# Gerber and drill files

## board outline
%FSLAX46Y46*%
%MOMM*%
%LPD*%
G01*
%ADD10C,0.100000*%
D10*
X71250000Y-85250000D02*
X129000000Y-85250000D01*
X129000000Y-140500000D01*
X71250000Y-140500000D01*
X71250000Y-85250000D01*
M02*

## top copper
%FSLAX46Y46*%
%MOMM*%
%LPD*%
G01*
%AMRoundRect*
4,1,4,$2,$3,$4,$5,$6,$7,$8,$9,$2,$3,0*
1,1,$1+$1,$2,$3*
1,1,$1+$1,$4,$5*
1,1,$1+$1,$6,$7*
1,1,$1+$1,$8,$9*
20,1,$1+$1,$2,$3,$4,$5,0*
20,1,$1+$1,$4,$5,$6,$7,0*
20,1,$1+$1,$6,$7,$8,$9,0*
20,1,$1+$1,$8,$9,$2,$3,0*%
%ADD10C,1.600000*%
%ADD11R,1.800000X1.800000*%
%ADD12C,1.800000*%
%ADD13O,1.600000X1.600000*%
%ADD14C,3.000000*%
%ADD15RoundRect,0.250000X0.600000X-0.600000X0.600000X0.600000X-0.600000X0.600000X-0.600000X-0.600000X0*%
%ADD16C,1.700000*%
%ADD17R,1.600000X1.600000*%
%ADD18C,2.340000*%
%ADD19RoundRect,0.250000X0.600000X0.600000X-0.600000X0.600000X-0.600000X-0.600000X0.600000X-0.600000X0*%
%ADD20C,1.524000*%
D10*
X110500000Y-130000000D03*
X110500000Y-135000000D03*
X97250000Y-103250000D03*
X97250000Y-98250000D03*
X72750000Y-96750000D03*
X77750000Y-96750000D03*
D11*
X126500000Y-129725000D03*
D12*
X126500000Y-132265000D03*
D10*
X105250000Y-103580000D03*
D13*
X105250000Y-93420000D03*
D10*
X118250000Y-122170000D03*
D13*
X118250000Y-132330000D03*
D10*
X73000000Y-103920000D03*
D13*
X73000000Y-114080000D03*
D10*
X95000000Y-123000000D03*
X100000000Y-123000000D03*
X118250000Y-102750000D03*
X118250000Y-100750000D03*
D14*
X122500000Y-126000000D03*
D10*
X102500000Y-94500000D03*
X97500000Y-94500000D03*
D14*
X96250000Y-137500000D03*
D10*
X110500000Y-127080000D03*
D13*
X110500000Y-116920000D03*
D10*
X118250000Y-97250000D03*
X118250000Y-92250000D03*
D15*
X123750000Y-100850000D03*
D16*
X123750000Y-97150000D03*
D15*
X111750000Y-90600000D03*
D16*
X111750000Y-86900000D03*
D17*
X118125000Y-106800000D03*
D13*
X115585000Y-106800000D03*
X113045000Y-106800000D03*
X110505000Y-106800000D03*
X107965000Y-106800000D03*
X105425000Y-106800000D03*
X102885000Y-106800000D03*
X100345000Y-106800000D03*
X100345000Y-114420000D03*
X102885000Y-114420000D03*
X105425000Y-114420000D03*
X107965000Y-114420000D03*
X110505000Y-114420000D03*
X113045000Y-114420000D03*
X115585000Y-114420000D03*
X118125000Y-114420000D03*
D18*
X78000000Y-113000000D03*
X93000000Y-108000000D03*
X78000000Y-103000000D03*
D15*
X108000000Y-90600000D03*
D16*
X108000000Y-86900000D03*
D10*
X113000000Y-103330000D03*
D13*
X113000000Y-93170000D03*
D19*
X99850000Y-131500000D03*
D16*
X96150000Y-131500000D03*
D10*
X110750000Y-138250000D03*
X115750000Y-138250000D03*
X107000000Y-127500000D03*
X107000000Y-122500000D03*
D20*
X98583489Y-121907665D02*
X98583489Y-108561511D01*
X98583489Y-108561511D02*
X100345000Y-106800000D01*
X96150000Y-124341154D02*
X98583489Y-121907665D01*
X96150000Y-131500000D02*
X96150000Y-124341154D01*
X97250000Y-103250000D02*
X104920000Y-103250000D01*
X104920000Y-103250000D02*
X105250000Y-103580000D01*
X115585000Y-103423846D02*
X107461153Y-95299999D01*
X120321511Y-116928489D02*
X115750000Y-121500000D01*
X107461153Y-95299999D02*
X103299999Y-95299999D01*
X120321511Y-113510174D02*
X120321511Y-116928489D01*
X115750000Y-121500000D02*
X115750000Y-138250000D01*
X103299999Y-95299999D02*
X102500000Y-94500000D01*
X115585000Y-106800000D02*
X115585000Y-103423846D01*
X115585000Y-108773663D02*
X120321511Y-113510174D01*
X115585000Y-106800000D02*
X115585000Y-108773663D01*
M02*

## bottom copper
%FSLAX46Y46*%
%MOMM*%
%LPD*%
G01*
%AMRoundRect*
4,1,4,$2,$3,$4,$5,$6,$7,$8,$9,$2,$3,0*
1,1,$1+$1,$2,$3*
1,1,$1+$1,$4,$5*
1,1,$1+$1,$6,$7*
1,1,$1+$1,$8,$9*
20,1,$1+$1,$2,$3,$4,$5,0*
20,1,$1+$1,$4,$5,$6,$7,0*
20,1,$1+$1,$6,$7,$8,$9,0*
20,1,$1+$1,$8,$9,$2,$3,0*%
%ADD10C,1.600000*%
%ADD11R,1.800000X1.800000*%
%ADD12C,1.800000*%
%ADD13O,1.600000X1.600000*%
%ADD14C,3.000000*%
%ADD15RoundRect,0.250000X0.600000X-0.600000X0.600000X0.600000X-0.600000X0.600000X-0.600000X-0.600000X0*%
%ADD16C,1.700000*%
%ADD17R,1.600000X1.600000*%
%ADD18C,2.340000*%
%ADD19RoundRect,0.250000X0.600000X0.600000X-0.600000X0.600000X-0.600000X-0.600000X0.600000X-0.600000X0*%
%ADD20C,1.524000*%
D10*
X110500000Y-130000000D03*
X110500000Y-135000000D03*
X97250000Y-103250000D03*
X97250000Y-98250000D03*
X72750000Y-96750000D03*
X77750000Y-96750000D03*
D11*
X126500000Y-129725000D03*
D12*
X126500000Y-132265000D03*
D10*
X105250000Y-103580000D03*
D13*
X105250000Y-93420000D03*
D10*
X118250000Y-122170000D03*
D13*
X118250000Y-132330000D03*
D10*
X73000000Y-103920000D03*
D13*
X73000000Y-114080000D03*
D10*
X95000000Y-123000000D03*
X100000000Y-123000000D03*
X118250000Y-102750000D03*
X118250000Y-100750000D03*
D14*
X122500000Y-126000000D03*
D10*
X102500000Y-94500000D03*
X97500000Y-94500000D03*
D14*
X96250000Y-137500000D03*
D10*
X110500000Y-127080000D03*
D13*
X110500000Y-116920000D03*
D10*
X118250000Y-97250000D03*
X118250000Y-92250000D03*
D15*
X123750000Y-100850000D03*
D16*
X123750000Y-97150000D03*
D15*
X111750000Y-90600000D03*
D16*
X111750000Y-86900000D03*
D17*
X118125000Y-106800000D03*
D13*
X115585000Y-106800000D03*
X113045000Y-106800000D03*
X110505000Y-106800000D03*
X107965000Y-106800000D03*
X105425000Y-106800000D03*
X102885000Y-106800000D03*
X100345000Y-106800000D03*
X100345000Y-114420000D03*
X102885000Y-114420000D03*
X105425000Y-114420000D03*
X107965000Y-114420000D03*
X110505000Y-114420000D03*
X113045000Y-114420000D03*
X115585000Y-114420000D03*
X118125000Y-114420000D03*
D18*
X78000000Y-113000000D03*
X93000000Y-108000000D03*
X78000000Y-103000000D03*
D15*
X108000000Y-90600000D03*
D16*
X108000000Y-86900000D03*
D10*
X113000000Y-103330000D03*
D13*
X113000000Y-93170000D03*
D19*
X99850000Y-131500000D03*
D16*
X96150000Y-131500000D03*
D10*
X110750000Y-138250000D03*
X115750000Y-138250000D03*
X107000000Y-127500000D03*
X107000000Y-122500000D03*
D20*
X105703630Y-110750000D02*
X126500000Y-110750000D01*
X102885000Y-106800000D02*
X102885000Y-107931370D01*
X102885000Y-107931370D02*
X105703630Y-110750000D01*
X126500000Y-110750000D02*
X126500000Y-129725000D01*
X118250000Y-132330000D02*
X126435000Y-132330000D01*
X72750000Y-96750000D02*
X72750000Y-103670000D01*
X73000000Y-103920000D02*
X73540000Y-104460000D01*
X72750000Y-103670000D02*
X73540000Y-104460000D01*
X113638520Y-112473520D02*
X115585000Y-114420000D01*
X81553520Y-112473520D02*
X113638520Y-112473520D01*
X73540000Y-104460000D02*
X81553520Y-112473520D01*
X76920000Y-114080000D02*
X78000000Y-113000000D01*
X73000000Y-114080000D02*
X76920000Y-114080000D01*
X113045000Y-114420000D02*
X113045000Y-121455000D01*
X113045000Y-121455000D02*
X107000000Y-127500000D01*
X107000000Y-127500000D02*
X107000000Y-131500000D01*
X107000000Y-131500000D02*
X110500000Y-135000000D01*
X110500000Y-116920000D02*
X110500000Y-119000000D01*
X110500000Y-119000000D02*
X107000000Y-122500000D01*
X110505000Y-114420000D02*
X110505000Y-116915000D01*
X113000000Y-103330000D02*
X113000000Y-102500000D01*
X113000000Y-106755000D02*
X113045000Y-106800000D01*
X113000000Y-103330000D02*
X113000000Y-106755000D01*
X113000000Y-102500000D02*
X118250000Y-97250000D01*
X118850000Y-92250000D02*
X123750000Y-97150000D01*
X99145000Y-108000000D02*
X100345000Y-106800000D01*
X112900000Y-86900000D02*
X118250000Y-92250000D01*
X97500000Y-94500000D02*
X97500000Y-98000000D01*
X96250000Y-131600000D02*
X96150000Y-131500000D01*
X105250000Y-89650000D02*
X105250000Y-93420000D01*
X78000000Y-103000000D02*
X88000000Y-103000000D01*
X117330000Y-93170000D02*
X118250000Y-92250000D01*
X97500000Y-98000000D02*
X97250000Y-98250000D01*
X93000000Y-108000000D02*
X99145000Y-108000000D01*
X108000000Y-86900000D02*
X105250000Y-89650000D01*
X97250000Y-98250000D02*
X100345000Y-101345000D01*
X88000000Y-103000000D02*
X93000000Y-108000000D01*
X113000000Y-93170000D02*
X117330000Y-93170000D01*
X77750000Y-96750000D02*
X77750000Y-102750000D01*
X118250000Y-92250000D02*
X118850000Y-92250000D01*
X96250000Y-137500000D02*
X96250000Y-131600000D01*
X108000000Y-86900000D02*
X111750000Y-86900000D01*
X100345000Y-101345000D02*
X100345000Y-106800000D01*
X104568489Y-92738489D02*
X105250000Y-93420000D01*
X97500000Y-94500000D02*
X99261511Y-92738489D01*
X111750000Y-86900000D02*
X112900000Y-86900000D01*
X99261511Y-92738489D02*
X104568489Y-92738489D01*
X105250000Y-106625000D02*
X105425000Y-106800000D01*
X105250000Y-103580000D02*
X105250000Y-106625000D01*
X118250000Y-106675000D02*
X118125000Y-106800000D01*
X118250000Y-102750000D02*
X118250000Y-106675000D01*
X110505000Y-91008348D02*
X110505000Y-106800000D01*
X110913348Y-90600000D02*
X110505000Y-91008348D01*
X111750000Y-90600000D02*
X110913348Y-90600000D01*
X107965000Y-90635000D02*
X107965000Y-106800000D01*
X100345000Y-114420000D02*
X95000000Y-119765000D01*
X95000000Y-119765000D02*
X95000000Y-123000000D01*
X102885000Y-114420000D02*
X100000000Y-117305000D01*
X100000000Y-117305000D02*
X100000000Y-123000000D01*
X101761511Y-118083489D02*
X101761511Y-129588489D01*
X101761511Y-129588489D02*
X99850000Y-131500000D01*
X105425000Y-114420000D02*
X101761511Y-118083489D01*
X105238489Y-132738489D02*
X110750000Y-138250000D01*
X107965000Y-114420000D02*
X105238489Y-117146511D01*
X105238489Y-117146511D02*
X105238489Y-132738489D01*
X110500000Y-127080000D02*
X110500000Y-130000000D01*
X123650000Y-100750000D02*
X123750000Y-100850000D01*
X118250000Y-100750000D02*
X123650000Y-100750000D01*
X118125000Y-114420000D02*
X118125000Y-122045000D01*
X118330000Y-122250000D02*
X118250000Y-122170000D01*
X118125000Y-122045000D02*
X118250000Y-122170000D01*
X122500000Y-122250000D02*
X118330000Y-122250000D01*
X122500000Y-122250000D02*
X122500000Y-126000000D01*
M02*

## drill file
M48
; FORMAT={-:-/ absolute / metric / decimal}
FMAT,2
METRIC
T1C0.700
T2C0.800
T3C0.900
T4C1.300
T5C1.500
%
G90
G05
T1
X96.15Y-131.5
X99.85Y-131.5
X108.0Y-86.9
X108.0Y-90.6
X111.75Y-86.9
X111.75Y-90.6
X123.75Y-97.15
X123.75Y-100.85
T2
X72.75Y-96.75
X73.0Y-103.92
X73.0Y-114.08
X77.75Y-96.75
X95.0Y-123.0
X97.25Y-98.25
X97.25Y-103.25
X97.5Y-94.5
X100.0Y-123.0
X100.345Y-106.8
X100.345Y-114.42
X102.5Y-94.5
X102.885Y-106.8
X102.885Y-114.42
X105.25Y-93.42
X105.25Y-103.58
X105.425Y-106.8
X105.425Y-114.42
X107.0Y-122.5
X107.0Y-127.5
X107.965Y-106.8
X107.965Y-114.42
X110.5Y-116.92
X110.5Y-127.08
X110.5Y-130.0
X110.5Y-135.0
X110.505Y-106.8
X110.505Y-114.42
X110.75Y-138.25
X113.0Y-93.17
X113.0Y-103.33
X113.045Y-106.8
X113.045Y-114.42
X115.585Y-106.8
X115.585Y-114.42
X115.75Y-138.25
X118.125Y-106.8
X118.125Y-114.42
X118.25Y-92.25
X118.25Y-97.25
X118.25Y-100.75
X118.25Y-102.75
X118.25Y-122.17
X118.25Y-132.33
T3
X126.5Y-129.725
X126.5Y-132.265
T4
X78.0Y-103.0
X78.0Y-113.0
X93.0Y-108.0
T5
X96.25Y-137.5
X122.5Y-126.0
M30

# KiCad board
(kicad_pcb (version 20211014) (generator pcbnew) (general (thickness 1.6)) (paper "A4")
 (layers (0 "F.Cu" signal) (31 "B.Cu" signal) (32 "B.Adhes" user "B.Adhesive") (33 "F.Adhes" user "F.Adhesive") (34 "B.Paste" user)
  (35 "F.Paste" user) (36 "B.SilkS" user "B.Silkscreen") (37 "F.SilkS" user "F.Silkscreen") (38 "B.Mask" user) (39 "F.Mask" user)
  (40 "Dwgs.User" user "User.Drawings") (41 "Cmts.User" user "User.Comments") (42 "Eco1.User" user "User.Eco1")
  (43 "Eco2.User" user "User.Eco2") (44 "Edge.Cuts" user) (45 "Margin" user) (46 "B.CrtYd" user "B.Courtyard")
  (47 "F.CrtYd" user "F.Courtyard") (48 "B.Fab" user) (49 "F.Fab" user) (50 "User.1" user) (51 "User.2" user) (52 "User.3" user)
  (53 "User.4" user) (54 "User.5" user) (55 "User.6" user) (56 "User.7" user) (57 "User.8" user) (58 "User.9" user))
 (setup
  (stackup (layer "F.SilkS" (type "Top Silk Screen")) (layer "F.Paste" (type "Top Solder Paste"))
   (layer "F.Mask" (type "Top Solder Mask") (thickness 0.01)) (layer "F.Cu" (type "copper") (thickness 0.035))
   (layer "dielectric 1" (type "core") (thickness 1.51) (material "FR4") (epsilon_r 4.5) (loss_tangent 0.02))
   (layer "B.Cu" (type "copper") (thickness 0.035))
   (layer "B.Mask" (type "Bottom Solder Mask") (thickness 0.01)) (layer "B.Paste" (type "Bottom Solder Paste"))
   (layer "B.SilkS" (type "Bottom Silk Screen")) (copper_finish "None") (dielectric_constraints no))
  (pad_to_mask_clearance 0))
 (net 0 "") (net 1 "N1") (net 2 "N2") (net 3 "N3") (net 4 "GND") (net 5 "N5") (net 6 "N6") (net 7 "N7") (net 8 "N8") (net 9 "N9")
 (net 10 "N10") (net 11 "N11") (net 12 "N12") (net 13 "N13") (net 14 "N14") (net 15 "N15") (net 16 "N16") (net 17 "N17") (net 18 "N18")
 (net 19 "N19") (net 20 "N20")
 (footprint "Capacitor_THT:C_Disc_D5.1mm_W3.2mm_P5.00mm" (layer "F.Cu") (at 110.5 130 -90)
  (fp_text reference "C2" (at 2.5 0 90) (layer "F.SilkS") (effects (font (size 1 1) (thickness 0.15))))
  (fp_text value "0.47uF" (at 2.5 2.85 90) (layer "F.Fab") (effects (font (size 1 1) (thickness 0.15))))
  (pad "1" thru_hole circle (at 0 0 270) (size 1.6 1.6) (drill 0.8) (layers *.Cu *.Mask) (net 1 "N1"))
  (pad "2" thru_hole circle (at 5 0 270) (size 1.6 1.6) (drill 0.8) (layers *.Cu *.Mask) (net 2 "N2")))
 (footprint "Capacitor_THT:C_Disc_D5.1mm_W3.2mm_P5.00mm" (layer "F.Cu") (at 97.25 103.25 90)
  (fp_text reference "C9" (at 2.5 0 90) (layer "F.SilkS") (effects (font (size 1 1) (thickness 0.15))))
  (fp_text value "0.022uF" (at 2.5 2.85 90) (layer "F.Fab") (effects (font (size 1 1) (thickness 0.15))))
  (pad "1" thru_hole circle (at 0 0 90) (size 1.6 1.6) (drill 0.8) (layers *.Cu *.Mask) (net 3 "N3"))
  (pad "2" thru_hole circle (at 5 0 90) (size 1.6 1.6) (drill 0.8) (layers *.Cu *.Mask) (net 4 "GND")))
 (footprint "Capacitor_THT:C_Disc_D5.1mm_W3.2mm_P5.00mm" (layer "F.Cu") (at 72.75 96.75)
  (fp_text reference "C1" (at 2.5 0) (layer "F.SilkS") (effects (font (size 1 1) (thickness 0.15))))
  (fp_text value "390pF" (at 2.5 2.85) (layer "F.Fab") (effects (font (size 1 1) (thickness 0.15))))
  (pad "1" thru_hole circle (at 0 0) (size 1.6 1.6) (drill 0.8) (layers *.Cu *.Mask) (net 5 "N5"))
  (pad "2" thru_hole circle (at 5 0) (size 1.6 1.6) (drill 0.8) (layers *.Cu *.Mask) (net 4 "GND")))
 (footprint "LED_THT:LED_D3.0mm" (layer "F.Cu") (at 126.5 129.725 -90)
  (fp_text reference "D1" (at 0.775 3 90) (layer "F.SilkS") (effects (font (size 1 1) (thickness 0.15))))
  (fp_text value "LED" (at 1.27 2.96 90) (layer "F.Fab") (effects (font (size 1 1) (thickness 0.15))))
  (pad "1" thru_hole rect (at 0 0 270) (size 1.8 1.8) (drill 0.9) (layers *.Cu *.Mask) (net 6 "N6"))
  (pad "2" thru_hole circle (at 2.54 0 270) (size 1.8 1.8) (drill 0.9) (layers *.Cu *.Mask) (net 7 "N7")))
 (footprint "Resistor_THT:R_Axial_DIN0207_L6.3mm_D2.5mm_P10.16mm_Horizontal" (layer "F.Cu") (at 105.25 103.58 90)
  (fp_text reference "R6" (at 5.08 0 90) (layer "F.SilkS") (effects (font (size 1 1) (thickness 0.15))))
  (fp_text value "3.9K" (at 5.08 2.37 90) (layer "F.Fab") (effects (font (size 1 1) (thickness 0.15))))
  (pad "1" thru_hole circle (at 0 0 90) (size 1.6 1.6) (drill 0.8) (layers *.Cu *.Mask) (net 3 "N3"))
  (pad "2" thru_hole oval (at 10.16 0 90) (size 1.6 1.6) (drill 0.8) (layers *.Cu *.Mask) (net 4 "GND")))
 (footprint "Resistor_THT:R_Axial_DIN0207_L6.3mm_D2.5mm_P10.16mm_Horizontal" (layer "F.Cu") (at 118.25 122.17 -90)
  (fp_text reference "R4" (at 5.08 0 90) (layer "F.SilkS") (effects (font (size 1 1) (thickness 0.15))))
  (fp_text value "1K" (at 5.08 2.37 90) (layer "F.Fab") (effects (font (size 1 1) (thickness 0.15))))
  (pad "1" thru_hole circle (at 0 0 270) (size 1.6 1.6) (drill 0.8) (layers *.Cu *.Mask) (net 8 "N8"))
  (pad "2" thru_hole oval (at 10.16 0 270) (size 1.6 1.6) (drill 0.8) (layers *.Cu *.Mask) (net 7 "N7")))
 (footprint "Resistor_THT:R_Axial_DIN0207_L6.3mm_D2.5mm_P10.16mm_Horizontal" (layer "F.Cu") (at 73 103.92 -90)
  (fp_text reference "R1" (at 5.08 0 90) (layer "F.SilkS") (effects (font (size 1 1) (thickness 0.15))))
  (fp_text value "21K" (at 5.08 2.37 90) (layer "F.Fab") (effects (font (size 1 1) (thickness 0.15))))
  (pad "1" thru_hole circle (at 0 0 270) (size 1.6 1.6) (drill 0.8) (layers *.Cu *.Mask) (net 5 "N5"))
  (pad "2" thru_hole oval (at 10.16 0 270) (size 1.6 1.6) (drill 0.8) (layers *.Cu *.Mask) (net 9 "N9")))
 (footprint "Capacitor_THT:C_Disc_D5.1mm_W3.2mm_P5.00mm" (layer "F.Cu") (at 95 123)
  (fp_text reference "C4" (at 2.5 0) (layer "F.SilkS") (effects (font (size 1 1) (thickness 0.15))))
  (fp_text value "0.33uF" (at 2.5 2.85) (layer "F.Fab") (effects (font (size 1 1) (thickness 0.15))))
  (pad "1" thru_hole circle (at 0 0) (size 1.6 1.6) (drill 0.8) (layers *.Cu *.Mask) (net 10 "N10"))
  (pad "2" thru_hole circle (at 5 0) (size 1.6 1.6) (drill 0.8) (layers *.Cu *.Mask) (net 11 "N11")))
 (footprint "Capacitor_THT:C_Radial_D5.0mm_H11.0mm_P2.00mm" (layer "F.Cu") (at 118.25 102.75 90)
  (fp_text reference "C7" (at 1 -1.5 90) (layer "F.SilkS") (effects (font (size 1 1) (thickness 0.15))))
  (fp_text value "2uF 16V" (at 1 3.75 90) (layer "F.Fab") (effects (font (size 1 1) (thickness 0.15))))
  (pad "1" thru_hole circle (at 0 0 90) (size 1.6 1.6) (drill 0.8) (layers *.Cu *.Mask) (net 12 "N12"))
  (pad "2" thru_hole circle (at 2 0 90) (size 1.6 1.6) (drill 0.8) (layers *.Cu *.Mask) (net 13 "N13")))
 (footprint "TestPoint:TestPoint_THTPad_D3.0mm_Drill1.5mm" (layer "F.Cu") (at 122.5 126)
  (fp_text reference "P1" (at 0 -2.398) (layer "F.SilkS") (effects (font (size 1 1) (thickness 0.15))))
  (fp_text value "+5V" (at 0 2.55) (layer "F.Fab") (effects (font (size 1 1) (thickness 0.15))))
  (pad "1" thru_hole circle (at 0 0) (size 3 3) (drill 1.5) (layers *.Cu *.Mask) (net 8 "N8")))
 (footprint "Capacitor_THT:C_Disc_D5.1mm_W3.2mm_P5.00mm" (layer "F.Cu") (at 102.5 94.5 180)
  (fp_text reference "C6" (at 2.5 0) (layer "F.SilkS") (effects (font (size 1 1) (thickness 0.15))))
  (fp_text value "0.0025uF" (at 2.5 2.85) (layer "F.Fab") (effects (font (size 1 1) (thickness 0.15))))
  (pad "1" thru_hole circle (at 0 0 180) (size 1.6 1.6) (drill 0.8) (layers *.Cu *.Mask) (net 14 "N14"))
  (pad "2" thru_hole circle (at 5 0 180) (size 1.6 1.6) (drill 0.8) (layers *.Cu *.Mask) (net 4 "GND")))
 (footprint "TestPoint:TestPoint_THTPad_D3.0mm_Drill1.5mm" (layer "F.Cu") (at 96.25 137.5)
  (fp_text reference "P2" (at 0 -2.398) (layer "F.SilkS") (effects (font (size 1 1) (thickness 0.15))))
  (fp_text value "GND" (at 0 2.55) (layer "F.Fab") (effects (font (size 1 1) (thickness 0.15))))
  (pad "1" thru_hole circle (at 0 0) (size 3 3) (drill 1.5) (layers *.Cu *.Mask) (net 4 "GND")))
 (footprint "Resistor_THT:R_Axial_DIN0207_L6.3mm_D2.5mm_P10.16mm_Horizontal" (layer "F.Cu") (at 110.5 127.08 90)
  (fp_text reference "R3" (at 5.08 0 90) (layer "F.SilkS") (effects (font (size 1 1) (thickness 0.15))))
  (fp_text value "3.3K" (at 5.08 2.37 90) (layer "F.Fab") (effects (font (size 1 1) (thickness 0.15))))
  (pad "1" thru_hole circle (at 0 0 90) (size 1.6 1.6) (drill 0.8) (layers *.Cu *.Mask) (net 1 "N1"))
  (pad "2" thru_hole oval (at 10.16 0 90) (size 1.6 1.6) (drill 0.8) (layers *.Cu *.Mask) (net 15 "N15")))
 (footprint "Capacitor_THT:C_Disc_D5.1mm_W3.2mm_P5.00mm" (layer "F.Cu") (at 118.25 97.25 90)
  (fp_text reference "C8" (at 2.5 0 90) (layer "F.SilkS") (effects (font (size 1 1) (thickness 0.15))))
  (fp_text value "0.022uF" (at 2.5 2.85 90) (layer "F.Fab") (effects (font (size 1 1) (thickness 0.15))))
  (pad "1" thru_hole circle (at 0 0 90) (size 1.6 1.6) (drill 0.8) (layers *.Cu *.Mask) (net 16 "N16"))
  (pad "2" thru_hole circle (at 5 0 90) (size 1.6 1.6) (drill 0.8) (layers *.Cu *.Mask) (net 4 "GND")))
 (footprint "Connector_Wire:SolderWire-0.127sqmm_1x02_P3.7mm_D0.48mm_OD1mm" (layer "F.Cu") (at 123.75 100.85 90)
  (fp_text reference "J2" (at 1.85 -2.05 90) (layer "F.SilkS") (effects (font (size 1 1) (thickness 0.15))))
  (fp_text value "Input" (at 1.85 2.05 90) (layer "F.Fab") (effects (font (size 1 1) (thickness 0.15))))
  (pad "1" thru_hole roundrect (at 0 0 90) (size 1.7 1.7) (drill 0.7) (layers *.Cu *.Mask) (roundrect_rratio 0.1470588235) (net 13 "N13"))
  (pad "2" thru_hole circle (at 3.7 0 90) (size 1.7 1.7) (drill 0.7) (layers *.Cu *.Mask) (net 4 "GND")))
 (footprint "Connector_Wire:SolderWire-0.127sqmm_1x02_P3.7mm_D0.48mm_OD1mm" (layer "F.Cu") (at 111.75 90.6 90)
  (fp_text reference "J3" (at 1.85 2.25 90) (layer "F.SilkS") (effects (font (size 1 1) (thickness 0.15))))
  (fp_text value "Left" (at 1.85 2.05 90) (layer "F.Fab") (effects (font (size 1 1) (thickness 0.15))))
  (pad "1" thru_hole roundrect (at 0 0 90) (size 1.7 1.7) (drill 0.7) (layers *.Cu *.Mask) (roundrect_rratio 0.1470588235) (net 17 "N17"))
  (pad "2" thru_hole circle (at 3.7 0 90) (size 1.7 1.7) (drill 0.7) (layers *.Cu *.Mask) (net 4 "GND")))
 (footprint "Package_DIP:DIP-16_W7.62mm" (layer "F.Cu") (at 118.125 106.8 -90)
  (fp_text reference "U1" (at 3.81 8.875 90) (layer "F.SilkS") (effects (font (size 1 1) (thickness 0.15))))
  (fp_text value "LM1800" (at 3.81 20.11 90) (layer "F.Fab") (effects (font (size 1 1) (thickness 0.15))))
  (pad "1" thru_hole rect (at 0 0 270) (size 1.6 1.6) (drill 0.8) (layers *.Cu *.Mask) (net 12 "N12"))
  (pad "2" thru_hole oval (at 0 2.54 270) (size 1.6 1.6) (drill 0.8) (layers *.Cu *.Mask) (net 14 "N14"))
  (pad "3" thru_hole oval (at 0 5.08 270) (size 1.6 1.6) (drill 0.8) (layers *.Cu *.Mask) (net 16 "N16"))
  (pad "4" thru_hole oval (at 0 7.62 270) (size 1.6 1.6) (drill 0.8) (layers *.Cu *.Mask) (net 17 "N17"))
  (pad "5" thru_hole oval (at 0 10.16 270) (size 1.6 1.6) (drill 0.8) (layers *.Cu *.Mask) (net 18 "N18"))
  (pad "6" thru_hole oval (at 0 12.7 270) (size 1.6 1.6) (drill 0.8) (layers *.Cu *.Mask) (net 3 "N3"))
  (pad "7" thru_hole oval (at 0 15.24 270) (size 1.6 1.6) (drill 0.8) (layers *.Cu *.Mask) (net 6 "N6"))
  (pad "8" thru_hole oval (at 0 17.78 270) (size 1.6 1.6) (drill 0.8) (layers *.Cu *.Mask) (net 4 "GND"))
  (pad "9" thru_hole oval (at 7.62 17.78 270) (size 1.6 1.6) (drill 0.8) (layers *.Cu *.Mask) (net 10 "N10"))
  (pad "10" thru_hole oval (at 7.62 15.24 270) (size 1.6 1.6) (drill 0.8) (layers *.Cu *.Mask) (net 11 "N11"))
  (pad "11" thru_hole oval (at 7.62 12.7 270) (size 1.6 1.6) (drill 0.8) (layers *.Cu *.Mask) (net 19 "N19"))
  (pad "12" thru_hole oval (at 7.62 10.16 270) (size 1.6 1.6) (drill 0.8) (layers *.Cu *.Mask) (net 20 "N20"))
  (pad "13" thru_hole oval (at 7.62 7.62 270) (size 1.6 1.6) (drill 0.8) (layers *.Cu *.Mask) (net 15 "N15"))
  (pad "14" thru_hole oval (at 7.62 5.08 270) (size 1.6 1.6) (drill 0.8) (layers *.Cu *.Mask) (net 2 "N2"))
  (pad "15" thru_hole oval (at 7.62 2.54 270) (size 1.6 1.6) (drill 0.8) (layers *.Cu *.Mask) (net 5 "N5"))
  (pad "16" thru_hole oval (at 7.62 0 270) (size 1.6 1.6) (drill 0.8) (layers *.Cu *.Mask) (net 8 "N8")))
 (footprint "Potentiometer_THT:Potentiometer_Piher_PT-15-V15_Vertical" (layer "F.Cu") (at 78 113)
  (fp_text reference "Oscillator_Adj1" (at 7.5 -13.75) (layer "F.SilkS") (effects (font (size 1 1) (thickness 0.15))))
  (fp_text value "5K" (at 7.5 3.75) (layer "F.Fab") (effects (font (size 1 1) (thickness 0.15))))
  (pad "1" thru_hole circle (at 0 0) (size 2.34 2.34) (drill 1.3) (layers *.Cu *.Mask) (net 9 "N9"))
  (pad "2" thru_hole circle (at 15 -5) (size 2.34 2.34) (drill 1.3) (layers *.Cu *.Mask) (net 4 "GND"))
  (pad "3" thru_hole circle (at 0 -10) (size 2.34 2.34) (drill 1.3) (layers *.Cu *.Mask) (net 4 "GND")))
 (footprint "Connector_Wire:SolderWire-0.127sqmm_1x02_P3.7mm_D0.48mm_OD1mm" (layer "F.Cu") (at 108 90.6 90)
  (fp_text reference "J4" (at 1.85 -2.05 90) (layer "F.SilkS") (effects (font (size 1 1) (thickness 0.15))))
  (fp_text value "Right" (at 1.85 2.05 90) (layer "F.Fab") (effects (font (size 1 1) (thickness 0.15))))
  (pad "1" thru_hole roundrect (at 0 0 90) (size 1.7 1.7) (drill 0.7) (layers *.Cu *.Mask) (roundrect_rratio 0.1470588235) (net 18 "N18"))
  (pad "2" thru_hole circle (at 3.7 0 90) (size 1.7 1.7) (drill 0.7) (layers *.Cu *.Mask) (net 4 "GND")))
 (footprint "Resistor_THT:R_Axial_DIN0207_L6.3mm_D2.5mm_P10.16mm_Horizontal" (layer "F.Cu") (at 113 103.33 90)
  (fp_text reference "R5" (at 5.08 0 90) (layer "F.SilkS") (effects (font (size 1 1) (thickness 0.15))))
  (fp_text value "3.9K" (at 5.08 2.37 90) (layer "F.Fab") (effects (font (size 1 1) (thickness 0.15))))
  (pad "1" thru_hole circle (at 0 0 90) (size 1.6 1.6) (drill 0.8) (layers *.Cu *.Mask) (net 16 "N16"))
  (pad "2" thru_hole oval (at 10.16 0 90) (size 1.6 1.6) (drill 0.8) (layers *.Cu *.Mask) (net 4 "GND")))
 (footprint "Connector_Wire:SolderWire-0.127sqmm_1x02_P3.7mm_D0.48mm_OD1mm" (layer "F.Cu") (at 99.85 131.5 180)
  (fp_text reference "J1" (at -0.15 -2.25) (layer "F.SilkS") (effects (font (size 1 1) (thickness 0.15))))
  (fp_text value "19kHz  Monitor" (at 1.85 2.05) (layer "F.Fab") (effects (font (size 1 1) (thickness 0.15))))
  (pad "1" thru_hole roundrect (at 0 0 180) (size 1.7 1.7) (drill 0.7) (layers *.Cu *.Mask) (roundrect_rratio 0.1470588235) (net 19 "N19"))
  (pad "2" thru_hole circle (at 3.7 0 180) (size 1.7 1.7) (drill 0.7) (layers *.Cu *.Mask) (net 4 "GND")))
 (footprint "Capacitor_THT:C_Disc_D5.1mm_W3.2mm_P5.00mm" (layer "F.Cu") (at 110.75 138.25)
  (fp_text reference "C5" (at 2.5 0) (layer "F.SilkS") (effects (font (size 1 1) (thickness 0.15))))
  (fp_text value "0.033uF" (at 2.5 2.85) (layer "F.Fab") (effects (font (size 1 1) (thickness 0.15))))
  (pad "1" thru_hole circle (at 0 0) (size 1.6 1.6) (drill 0.8) (layers *.Cu *.Mask) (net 20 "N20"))
  (pad "2" thru_hole circle (at 5 0) (size 1.6 1.6) (drill 0.8) (layers *.Cu *.Mask) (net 14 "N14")))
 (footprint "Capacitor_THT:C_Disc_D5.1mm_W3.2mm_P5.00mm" (layer "F.Cu") (at 107 127.5 90)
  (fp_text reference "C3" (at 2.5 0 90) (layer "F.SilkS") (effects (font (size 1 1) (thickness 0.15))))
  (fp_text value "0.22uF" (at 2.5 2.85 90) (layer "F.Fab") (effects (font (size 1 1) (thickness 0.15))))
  (pad "1" thru_hole circle (at 0 0 90) (size 1.6 1.6) (drill 0.8) (layers *.Cu *.Mask) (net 2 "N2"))
  (pad "2" thru_hole circle (at 5 0 90) (size 1.6 1.6) (drill 0.8) (layers *.Cu *.Mask) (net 15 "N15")))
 (gr_rect (start 129 85.25) (end 71.25 140.5) (layer "Edge.Cuts") (width 0.1) (fill none))
 (segment (start 105.70363 110.75) (end 126.5 110.75) (width 1.524) (layer "B.Cu") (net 6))
 (segment (start 102.885 106.8) (end 102.885 107.93137) (width 1.524) (layer "B.Cu") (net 6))
 (segment (start 102.885 107.93137) (end 105.70363 110.75) (width 1.524) (layer "B.Cu") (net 6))
 (segment (start 126.5 110.75) (end 126.5 129.725) (width 1.524) (layer "B.Cu") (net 6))
 (segment (start 118.25 132.33) (end 126.435 132.33) (width 1.524) (layer "B.Cu") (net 7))
 (segment (start 72.75 96.75) (end 72.75 103.67) (width 1.524) (layer "B.Cu") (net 5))
 (segment (start 73 103.92) (end 73.54 104.46) (width 1.524) (layer "B.Cu") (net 5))
 (segment (start 72.75 103.67) (end 73.54 104.46) (width 1.524) (layer "B.Cu") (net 5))
 (segment (start 113.63852 112.47352) (end 115.585 114.42) (width 1.524) (layer "B.Cu") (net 5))
 (segment (start 81.55352 112.47352) (end 113.63852 112.47352) (width 1.524) (layer "B.Cu") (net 5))
 (segment (start 73.54 104.46) (end 81.55352 112.47352) (width 1.524) (layer "B.Cu") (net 5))
 (segment (start 76.92 114.08) (end 78 113) (width 1.524) (layer "B.Cu") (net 9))
 (segment (start 73 114.08) (end 76.92 114.08) (width 1.524) (layer "B.Cu") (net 9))
 (segment (start 113.045 114.42) (end 113.045 121.455) (width 1.524) (layer "B.Cu") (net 2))
 (segment (start 113.045 121.455) (end 107 127.5) (width 1.524) (layer "B.Cu") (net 2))
 (segment (start 107 127.5) (end 107 131.5) (width 1.524) (layer "B.Cu") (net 2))
 (segment (start 107 131.5) (end 110.5 135) (width 1.524) (layer "B.Cu") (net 2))
 (segment (start 110.5 116.92) (end 110.5 119) (width 1.524) (layer "B.Cu") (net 15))
 (segment (start 110.5 119) (end 107 122.5) (width 1.524) (layer "B.Cu") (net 15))
 (segment (start 110.505 114.42) (end 110.505 116.915) (width 1.524) (layer "B.Cu") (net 15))
 (segment (start 113 103.33) (end 113 102.5) (width 1.524) (layer "B.Cu") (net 16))
 (segment (start 113 106.755) (end 113.045 106.8) (width 1.524) (layer "B.Cu") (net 16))
 (segment (start 113 103.33) (end 113 106.755) (width 1.524) (layer "B.Cu") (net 16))
 (segment (start 113 102.5) (end 118.25 97.25) (width 1.524) (layer "B.Cu") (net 16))
 (segment (start 98.583489 121.907665) (end 98.583489 108.561511) (width 1.524) (layer "F.Cu") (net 4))
 (segment (start 98.583489 108.561511) (end 100.345 106.8) (width 1.524) (layer "F.Cu") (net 4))
 (segment (start 96.15 124.341154) (end 98.583489 121.907665) (width 1.524) (layer "F.Cu") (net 4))
 (segment (start 96.15 131.5) (end 96.15 124.341154) (width 1.524) (layer "F.Cu") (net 4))
 (segment (start 118.85 92.25) (end 123.75 97.15) (width 1.524) (layer "B.Cu") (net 4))
 (segment (start 99.145 108) (end 100.345 106.8) (width 1.524) (layer "B.Cu") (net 4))
 (segment (start 112.9 86.9) (end 118.25 92.25) (width 1.524) (layer "B.Cu") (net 4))
 (segment (start 97.5 94.5) (end 97.5 98) (width 1.524) (layer "B.Cu") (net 4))
 (segment (start 96.25 131.6) (end 96.15 131.5) (width 1.524) (layer "B.Cu") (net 4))
 (segment (start 105.25 89.65) (end 105.25 93.42) (width 1.524) (layer "B.Cu") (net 4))
 (segment (start 78 103) (end 88 103) (width 1.524) (layer "B.Cu") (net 4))
 (segment (start 117.33 93.17) (end 118.25 92.25) (width 1.524) (layer "B.Cu") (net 4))
 (segment (start 97.5 98) (end 97.25 98.25) (width 1.524) (layer "B.Cu") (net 4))
 (segment (start 93 108) (end 99.145 108) (width 1.524) (layer "B.Cu") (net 4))
 (segment (start 108 86.9) (end 105.25 89.65) (width 1.524) (layer "B.Cu") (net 4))
 (segment (start 97.25 98.25) (end 100.345 101.345) (width 1.524) (layer "B.Cu") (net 4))
 (segment (start 88 103) (end 93 108) (width 1.524) (layer "B.Cu") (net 4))
 (segment (start 113 93.17) (end 117.33 93.17) (width 1.524) (layer "B.Cu") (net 4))
 (segment (start 77.75 96.75) (end 77.75 102.75) (width 1.524) (layer "B.Cu") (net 4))
 (segment (start 118.25 92.25) (end 118.85 92.25) (width 1.524) (layer "B.Cu") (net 4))
 (segment (start 96.25 137.5) (end 96.25 131.6) (width 1.524) (layer "B.Cu") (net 4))
 (segment (start 108 86.9) (end 111.75 86.9) (width 1.524) (layer "B.Cu") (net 4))
 (segment (start 100.345 101.345) (end 100.345 106.8) (width 1.524) (layer "B.Cu") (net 4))
 (segment (start 104.568489 92.738489) (end 105.25 93.42) (width 1.524) (layer "B.Cu") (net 4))
 (segment (start 97.5 94.5) (end 99.261511 92.738489) (width 1.524) (layer "B.Cu") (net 4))
 (segment (start 111.75 86.9) (end 112.9 86.9) (width 1.524) (layer "B.Cu") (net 4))
 (segment (start 99.261511 92.738489) (end 104.568489 92.738489) (width 1.524) (layer "B.Cu") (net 4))
 (segment (start 97.25 103.25) (end 104.92 103.25) (width 1.524) (layer "F.Cu") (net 3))
 (segment (start 104.92 103.25) (end 105.25 103.58) (width 1.524) (layer "F.Cu") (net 3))
 (segment (start 105.25 106.625) (end 105.425 106.8) (width 1.524) (layer "B.Cu") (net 3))
 (segment (start 105.25 103.58) (end 105.25 106.625) (width 1.524) (layer "B.Cu") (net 3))
 (segment (start 118.25 106.675) (end 118.125 106.8) (width 1.524) (layer "B.Cu") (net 12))
 (segment (start 118.25 102.75) (end 118.25 106.675) (width 1.524) (layer "B.Cu") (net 12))
 (segment (start 115.585 103.423846) (end 107.461153 95.299999) (width 1.524) (layer "F.Cu") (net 14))
 (segment (start 120.321511 116.928489) (end 115.75 121.5) (width 1.524) (layer "F.Cu") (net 14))
 (segment (start 107.461153 95.299999) (end 103.299999 95.299999) (width 1.524) (layer "F.Cu") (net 14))
 (segment (start 120.321511 113.510174) (end 120.321511 116.928489) (width 1.524) (layer "F.Cu") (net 14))
 (segment (start 115.75 121.5) (end 115.75 138.25) (width 1.524) (layer "F.Cu") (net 14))
 (segment (start 103.299999 95.299999) (end 102.5 94.5) (width 1.524) (layer "F.Cu") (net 14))
 (segment (start 115.585 106.8) (end 115.585 103.423846) (width 1.524) (layer "F.Cu") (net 14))
 (segment (start 115.585 108.773663) (end 120.321511 113.510174) (width 1.524) (layer "F.Cu") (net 14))
 (segment (start 115.585 106.8) (end 115.585 108.773663) (width 1.524) (layer "F.Cu") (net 14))
 (segment (start 110.505 91.008348) (end 110.505 106.8) (width 1.524) (layer "B.Cu") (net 17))
 (segment (start 110.913348 90.6) (end 110.505 91.008348) (width 1.524) (layer "B.Cu") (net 17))
 (segment (start 111.75 90.6) (end 110.913348 90.6) (width 1.524) (layer "B.Cu") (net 17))
 (segment (start 107.965 90.635) (end 107.965 106.8) (width 1.524) (layer "B.Cu") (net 18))
 (segment (start 100.345 114.42) (end 95 119.765) (width 1.524) (layer "B.Cu") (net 10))
 (segment (start 95 119.765) (end 95 123) (width 1.524) (layer "B.Cu") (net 10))
 (segment (start 102.885 114.42) (end 100 117.305) (width 1.524) (layer "B.Cu") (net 11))
 (segment (start 100 117.305) (end 100 123) (width 1.524) (layer "B.Cu") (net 11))
 (segment (start 101.761511 118.083489) (end 101.761511 129.588489) (width 1.524) (layer "B.Cu") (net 19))
 (segment (start 101.761511 129.588489) (end 99.85 131.5) (width 1.524) (layer "B.Cu") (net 19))
 (segment (start 105.425 114.42) (end 101.761511 118.083489) (width 1.524) (layer "B.Cu") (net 19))
 (segment (start 105.238489 132.738489) (end 110.75 138.25) (width 1.524) (layer "B.Cu") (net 20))
 (segment (start 107.965 114.42) (end 105.238489 117.146511) (width 1.524) (layer "B.Cu") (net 20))
 (segment (start 105.238489 117.146511) (end 105.238489 132.738489) (width 1.524) (layer "B.Cu") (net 20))
 (segment (start 110.5 127.08) (end 110.5 130) (width 1.524) (layer "B.Cu") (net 1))
 (segment (start 123.65 100.75) (end 123.75 100.85) (width 1.524) (layer "B.Cu") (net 13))
 (segment (start 118.25 100.75) (end 123.65 100.75) (width 1.524) (layer "B.Cu") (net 13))
 (segment (start 118.125 114.42) (end 118.125 122.045) (width 1.524) (layer "B.Cu") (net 8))
 (segment (start 118.33 122.25) (end 118.25 122.17) (width 1.524) (layer "B.Cu") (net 8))
 (segment (start 118.125 122.045) (end 118.25 122.17) (width 1.524) (layer "B.Cu") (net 8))
 (segment (start 122.5 122.25) (end 118.33 122.25) (width 1.524) (layer "B.Cu") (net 8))
 (segment (start 122.5 122.25) (end 122.5 126) (width 1.524) (layer "B.Cu") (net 8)))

